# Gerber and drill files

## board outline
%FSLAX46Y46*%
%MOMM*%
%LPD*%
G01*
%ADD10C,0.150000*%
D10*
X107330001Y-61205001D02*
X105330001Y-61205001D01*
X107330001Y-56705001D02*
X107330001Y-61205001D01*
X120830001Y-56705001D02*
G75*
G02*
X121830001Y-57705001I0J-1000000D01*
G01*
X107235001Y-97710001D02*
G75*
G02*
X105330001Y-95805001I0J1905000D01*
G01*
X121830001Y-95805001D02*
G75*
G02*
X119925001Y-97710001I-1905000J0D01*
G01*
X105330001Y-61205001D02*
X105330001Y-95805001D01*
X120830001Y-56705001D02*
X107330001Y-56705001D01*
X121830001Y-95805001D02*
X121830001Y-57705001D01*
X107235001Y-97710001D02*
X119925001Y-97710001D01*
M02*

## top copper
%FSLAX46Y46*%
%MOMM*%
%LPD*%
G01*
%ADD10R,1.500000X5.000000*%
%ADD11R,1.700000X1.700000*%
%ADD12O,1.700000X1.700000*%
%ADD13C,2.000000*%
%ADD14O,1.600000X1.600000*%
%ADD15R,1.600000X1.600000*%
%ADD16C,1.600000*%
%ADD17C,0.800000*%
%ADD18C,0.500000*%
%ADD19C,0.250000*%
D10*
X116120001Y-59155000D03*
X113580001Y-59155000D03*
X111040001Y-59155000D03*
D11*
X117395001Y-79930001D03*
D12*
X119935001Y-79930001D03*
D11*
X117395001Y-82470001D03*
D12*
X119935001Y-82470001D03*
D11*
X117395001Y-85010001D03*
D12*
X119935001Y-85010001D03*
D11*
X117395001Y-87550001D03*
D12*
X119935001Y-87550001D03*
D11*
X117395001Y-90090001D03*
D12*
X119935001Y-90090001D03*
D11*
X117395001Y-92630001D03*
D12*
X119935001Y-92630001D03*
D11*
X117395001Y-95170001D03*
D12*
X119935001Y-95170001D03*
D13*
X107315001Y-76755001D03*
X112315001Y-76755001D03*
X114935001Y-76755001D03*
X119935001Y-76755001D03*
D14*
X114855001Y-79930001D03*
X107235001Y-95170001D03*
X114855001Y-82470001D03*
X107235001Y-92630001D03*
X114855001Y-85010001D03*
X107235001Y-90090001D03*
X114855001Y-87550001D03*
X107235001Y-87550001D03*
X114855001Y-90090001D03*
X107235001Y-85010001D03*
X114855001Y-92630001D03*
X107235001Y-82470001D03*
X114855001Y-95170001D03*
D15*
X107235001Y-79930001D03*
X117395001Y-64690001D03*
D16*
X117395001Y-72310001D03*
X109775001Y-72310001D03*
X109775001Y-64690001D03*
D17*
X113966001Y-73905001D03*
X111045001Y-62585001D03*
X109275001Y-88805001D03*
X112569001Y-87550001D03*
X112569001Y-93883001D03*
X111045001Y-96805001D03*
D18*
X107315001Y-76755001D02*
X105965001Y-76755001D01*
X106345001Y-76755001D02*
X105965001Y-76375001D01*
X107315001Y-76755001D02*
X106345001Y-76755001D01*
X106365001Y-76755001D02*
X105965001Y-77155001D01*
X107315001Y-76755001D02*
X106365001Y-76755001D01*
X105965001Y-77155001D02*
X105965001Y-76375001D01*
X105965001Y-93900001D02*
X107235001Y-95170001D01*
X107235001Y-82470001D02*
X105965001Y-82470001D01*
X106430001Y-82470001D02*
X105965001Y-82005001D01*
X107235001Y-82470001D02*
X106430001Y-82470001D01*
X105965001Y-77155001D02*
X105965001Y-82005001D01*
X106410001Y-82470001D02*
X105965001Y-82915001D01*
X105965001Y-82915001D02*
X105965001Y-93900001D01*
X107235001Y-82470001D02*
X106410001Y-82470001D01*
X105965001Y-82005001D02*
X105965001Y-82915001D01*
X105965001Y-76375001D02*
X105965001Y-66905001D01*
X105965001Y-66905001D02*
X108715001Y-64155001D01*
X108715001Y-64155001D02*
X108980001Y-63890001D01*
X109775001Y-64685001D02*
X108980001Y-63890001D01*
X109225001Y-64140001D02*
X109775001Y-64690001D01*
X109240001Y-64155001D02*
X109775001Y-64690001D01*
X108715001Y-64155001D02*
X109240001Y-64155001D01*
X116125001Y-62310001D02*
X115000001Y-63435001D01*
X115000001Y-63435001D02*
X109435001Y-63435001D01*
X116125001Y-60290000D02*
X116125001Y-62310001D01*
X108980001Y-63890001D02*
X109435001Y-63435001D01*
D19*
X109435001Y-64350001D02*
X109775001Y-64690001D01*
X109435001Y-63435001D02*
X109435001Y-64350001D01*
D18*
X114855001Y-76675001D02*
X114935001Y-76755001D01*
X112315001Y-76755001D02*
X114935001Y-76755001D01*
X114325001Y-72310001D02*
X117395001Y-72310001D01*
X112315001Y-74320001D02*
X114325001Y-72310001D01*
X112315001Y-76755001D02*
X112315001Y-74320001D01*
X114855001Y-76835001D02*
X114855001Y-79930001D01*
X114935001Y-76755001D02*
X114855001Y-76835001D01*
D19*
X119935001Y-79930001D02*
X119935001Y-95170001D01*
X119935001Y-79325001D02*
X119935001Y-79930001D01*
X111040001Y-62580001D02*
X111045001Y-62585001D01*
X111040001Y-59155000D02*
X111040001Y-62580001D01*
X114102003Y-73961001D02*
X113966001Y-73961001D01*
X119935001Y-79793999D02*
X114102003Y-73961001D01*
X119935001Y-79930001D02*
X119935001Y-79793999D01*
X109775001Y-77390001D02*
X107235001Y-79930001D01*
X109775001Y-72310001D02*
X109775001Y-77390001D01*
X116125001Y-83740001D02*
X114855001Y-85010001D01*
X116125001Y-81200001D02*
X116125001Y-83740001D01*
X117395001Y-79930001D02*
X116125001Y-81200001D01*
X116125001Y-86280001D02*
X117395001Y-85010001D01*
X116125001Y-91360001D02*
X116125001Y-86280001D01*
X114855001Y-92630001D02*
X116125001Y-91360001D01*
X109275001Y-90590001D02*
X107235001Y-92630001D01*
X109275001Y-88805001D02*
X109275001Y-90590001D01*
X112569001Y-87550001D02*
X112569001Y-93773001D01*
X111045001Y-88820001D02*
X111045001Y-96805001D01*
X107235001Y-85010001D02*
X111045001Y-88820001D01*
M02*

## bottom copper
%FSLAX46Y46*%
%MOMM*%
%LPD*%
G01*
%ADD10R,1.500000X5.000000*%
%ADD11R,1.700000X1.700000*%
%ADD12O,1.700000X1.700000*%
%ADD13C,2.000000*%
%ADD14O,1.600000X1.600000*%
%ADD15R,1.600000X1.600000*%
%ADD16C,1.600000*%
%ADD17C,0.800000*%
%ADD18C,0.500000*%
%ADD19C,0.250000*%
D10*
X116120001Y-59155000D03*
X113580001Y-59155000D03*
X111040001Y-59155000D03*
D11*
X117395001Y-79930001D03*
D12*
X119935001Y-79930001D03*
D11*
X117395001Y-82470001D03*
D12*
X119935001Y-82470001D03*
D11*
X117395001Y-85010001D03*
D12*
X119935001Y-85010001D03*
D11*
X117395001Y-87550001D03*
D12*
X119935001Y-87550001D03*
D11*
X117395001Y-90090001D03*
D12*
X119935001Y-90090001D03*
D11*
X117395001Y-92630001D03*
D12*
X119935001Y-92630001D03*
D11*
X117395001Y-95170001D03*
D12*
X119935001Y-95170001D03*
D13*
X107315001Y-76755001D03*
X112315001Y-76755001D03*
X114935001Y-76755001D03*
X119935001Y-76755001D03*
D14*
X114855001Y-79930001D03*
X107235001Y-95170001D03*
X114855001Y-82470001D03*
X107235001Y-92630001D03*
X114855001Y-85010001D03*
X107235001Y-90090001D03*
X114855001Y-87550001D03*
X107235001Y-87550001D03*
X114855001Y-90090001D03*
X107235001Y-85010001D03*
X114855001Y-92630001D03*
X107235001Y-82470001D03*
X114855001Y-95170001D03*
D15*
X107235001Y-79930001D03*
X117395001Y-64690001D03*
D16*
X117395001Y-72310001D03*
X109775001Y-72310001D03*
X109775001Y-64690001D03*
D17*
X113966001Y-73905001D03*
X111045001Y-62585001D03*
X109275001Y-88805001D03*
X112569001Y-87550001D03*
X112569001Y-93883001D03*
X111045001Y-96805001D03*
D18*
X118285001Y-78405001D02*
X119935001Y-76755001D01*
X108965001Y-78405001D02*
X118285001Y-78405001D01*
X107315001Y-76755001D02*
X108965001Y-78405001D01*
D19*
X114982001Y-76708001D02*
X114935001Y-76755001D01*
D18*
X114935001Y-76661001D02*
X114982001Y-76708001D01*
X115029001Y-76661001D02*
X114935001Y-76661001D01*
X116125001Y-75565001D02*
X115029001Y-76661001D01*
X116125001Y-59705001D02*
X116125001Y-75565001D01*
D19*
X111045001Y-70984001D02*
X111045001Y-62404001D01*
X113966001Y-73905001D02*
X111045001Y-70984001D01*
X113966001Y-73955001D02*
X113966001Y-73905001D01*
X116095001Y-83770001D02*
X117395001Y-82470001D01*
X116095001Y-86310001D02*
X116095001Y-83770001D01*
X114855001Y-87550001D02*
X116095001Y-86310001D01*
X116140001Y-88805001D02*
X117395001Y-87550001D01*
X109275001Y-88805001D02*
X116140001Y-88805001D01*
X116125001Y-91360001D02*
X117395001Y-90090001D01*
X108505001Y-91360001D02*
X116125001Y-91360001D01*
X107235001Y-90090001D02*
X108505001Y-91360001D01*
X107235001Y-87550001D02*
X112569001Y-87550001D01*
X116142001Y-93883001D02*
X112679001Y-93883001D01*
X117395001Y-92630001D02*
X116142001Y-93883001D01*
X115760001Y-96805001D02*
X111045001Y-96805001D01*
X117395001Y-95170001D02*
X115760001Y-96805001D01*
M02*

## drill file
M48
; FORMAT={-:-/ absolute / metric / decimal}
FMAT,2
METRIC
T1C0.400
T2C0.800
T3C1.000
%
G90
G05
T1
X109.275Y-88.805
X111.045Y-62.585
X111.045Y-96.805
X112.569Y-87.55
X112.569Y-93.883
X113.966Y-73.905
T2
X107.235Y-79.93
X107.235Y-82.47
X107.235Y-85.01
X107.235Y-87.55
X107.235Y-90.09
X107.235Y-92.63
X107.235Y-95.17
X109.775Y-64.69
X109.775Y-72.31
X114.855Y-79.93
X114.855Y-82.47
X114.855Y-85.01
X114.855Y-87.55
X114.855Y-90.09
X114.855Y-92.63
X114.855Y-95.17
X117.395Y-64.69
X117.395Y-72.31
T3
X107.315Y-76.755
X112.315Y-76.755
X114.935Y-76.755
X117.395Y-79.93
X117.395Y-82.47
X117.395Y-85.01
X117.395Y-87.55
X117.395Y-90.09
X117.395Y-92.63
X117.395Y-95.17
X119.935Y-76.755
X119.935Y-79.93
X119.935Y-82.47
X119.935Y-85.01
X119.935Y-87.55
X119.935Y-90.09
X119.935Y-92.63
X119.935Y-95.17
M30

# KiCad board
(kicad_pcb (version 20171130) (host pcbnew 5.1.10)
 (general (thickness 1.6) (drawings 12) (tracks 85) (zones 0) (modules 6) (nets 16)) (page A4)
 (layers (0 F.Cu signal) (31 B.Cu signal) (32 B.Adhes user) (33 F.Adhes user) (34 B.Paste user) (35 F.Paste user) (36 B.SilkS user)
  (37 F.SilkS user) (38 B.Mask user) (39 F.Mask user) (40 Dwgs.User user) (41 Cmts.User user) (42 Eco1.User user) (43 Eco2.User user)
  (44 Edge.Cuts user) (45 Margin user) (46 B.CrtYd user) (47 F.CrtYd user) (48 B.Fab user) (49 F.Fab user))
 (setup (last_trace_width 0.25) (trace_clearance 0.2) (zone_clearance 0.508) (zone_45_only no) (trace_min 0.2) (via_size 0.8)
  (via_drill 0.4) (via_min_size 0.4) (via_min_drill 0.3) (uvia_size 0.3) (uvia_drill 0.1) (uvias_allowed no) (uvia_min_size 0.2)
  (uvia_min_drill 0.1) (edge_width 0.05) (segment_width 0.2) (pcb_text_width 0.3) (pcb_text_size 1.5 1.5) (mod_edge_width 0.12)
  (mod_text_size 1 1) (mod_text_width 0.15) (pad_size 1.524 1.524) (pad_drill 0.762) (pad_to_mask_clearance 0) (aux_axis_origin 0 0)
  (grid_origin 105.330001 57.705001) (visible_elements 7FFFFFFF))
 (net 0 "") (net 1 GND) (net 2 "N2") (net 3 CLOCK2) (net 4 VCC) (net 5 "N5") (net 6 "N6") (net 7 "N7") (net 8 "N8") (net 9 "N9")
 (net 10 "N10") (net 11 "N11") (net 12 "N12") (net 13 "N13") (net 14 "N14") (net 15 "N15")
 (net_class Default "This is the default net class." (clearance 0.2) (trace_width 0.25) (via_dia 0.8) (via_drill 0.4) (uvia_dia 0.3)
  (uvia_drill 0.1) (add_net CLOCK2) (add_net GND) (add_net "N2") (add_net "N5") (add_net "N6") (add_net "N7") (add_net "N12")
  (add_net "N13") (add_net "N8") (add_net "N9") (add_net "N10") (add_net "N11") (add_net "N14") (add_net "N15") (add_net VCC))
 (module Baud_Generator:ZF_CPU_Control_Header (layer F.Cu) (at 113.580001 59.155 180)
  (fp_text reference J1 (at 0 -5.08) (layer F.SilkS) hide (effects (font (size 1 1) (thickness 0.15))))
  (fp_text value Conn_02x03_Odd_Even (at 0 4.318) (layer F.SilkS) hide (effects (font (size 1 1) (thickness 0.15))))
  (pad 1 connect rect (at -2.54 0) (size 1.5 5) (layers F.Cu) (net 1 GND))
  (pad 3 connect rect (at 0 0) (size 1.5 5) (layers F.Cu) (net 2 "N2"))
  (pad 5 connect rect (at 2.54 0) (size 1.5 5) (layers F.Cu) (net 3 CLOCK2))
  (pad 2 connect rect (at -2.54 0) (size 1.5 5) (layers B.Cu) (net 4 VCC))
  (pad 4 connect rect (at 0 0) (size 1.5 5) (layers B.Cu) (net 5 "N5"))
  (pad 6 connect rect (at 2.54 0) (size 1.5 5) (layers B.Cu) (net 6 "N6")))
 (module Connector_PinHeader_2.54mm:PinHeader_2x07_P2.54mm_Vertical (layer F.Cu) (at 117.395001 79.930001)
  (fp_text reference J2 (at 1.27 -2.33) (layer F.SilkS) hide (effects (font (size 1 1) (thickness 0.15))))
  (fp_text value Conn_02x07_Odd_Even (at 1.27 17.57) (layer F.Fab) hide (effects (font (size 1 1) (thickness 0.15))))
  (pad 1 thru_hole rect (at 0 0) (size 1.7 1.7) (drill 1) (layers *.Cu *.Mask) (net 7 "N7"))
  (pad 2 thru_hole oval (at 2.54 0) (size 1.7 1.7) (drill 1) (layers *.Cu *.Mask) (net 3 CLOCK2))
  (pad 3 thru_hole rect (at 0 2.54) (size 1.7 1.7) (drill 1) (layers *.Cu *.Mask) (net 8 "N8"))
  (pad 4 thru_hole oval (at 2.54 2.54) (size 1.7 1.7) (drill 1) (layers *.Cu *.Mask) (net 3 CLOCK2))
  (pad 5 thru_hole rect (at 0 5.08) (size 1.7 1.7) (drill 1) (layers *.Cu *.Mask) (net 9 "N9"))
  (pad 6 thru_hole oval (at 2.54 5.08) (size 1.7 1.7) (drill 1) (layers *.Cu *.Mask) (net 3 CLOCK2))
  (pad 7 thru_hole rect (at 0 7.62) (size 1.7 1.7) (drill 1) (layers *.Cu *.Mask) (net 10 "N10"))
  (pad 8 thru_hole oval (at 2.54 7.62) (size 1.7 1.7) (drill 1) (layers *.Cu *.Mask) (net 3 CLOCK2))
  (pad 9 thru_hole rect (at 0 10.16) (size 1.7 1.7) (drill 1) (layers *.Cu *.Mask) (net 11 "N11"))
  (pad 10 thru_hole oval (at 2.54 10.16) (size 1.7 1.7) (drill 1) (layers *.Cu *.Mask) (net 3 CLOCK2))
  (pad 11 thru_hole rect (at 0 12.7) (size 1.7 1.7) (drill 1) (layers *.Cu *.Mask) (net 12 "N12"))
  (pad 12 thru_hole oval (at 2.54 12.7) (size 1.7 1.7) (drill 1) (layers *.Cu *.Mask) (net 3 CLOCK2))
  (pad 13 thru_hole rect (at 0 15.24) (size 1.7 1.7) (drill 1) (layers *.Cu *.Mask) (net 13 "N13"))
  (pad 14 thru_hole oval (at 2.54 15.24) (size 1.7 1.7) (drill 1) (layers *.Cu *.Mask) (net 3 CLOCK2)))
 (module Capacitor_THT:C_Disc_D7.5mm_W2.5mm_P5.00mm (layer F.Cu) (at 112.315001 76.755001 180)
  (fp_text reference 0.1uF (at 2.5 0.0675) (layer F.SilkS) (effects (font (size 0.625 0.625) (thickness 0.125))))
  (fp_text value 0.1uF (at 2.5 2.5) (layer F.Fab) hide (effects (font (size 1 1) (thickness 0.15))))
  (pad 2 thru_hole circle (at 5 0 180) (size 2 2) (drill 1) (layers *.Cu *.Mask) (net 1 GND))
  (pad 1 thru_hole circle (at 0 0 180) (size 2 2) (drill 1) (layers *.Cu *.Mask) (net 4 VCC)))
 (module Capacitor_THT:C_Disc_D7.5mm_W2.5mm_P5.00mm (layer F.Cu) (at 114.935001 76.755001)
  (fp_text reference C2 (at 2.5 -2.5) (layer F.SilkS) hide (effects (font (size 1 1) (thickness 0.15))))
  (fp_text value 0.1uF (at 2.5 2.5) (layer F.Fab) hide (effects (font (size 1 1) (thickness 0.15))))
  (pad 1 thru_hole circle (at 0 0) (size 2 2) (drill 1) (layers *.Cu *.Mask) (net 4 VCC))
  (pad 2 thru_hole circle (at 5 0) (size 2 2) (drill 1) (layers *.Cu *.Mask) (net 1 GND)))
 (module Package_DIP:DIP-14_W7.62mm (layer F.Cu) (at 107.235001 79.930001)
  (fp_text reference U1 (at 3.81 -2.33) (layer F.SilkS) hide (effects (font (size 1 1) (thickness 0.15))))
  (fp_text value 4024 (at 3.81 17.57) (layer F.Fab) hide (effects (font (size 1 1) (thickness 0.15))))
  (pad 14 thru_hole oval (at 7.62 0) (size 1.6 1.6) (drill 0.8) (layers *.Cu *.Mask) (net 4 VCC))
  (pad 7 thru_hole oval (at 0 15.24) (size 1.6 1.6) (drill 0.8) (layers *.Cu *.Mask) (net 1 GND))
  (pad 13 thru_hole oval (at 7.62 2.54) (size 1.6 1.6) (drill 0.8) (layers *.Cu *.Mask))
  (pad 6 thru_hole oval (at 0 12.7) (size 1.6 1.6) (drill 0.8) (layers *.Cu *.Mask) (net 10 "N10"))
  (pad 12 thru_hole oval (at 7.62 5.08) (size 1.6 1.6) (drill 0.8) (layers *.Cu *.Mask) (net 7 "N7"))
  (pad 5 thru_hole oval (at 0 10.16) (size 1.6 1.6) (drill 0.8) (layers *.Cu *.Mask) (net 11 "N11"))
  (pad 11 thru_hole oval (at 7.62 7.62) (size 1.6 1.6) (drill 0.8) (layers *.Cu *.Mask) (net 8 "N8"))
  (pad 4 thru_hole oval (at 0 7.62) (size 1.6 1.6) (drill 0.8) (layers *.Cu *.Mask) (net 12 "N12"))
  (pad 10 thru_hole oval (at 7.62 10.16) (size 1.6 1.6) (drill 0.8) (layers *.Cu *.Mask))
  (pad 3 thru_hole oval (at 0 5.08) (size 1.6 1.6) (drill 0.8) (layers *.Cu *.Mask) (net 13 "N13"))
  (pad 9 thru_hole oval (at 7.62 12.7) (size 1.6 1.6) (drill 0.8) (layers *.Cu *.Mask) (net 9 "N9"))
  (pad 2 thru_hole oval (at 0 2.54) (size 1.6 1.6) (drill 0.8) (layers *.Cu *.Mask) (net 1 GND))
  (pad 8 thru_hole oval (at 7.62 15.24) (size 1.6 1.6) (drill 0.8) (layers *.Cu *.Mask))
  (pad 1 thru_hole rect (at 0 0) (size 1.6 1.6) (drill 0.8) (layers *.Cu *.Mask) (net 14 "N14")))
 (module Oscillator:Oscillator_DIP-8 (layer F.Cu) (at 117.395001 64.690001 180)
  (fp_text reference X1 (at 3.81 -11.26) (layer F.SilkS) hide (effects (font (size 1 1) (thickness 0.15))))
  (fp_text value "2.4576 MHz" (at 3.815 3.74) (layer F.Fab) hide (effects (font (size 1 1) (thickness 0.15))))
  (pad 1 thru_hole rect (at 0 0 180) (size 1.6 1.6) (drill 0.8) (layers *.Cu *.Mask) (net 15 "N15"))
  (pad 8 thru_hole circle (at 0 -7.62 180) (size 1.6 1.6) (drill 0.8) (layers *.Cu *.Mask) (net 4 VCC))
  (pad 5 thru_hole circle (at 7.62 -7.62 180) (size 1.6 1.6) (drill 0.8) (layers *.Cu *.Mask) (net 14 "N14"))
  (pad 4 thru_hole circle (at 7.62 0 180) (size 1.6 1.6) (drill 0.8) (layers *.Cu *.Mask) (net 1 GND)))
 (gr_line (start 107.330001 61.205001) (end 105.330001 61.205001) (layer Edge.Cuts) (width 0.15))
 (gr_line (start 107.330001 56.705001) (end 107.330001 61.205001) (layer Edge.Cuts) (width 0.15))
 (gr_arc (start 120.830001 57.705001) (end 121.830001 57.705001) (angle -90) (layer Edge.Cuts) (width 0.15))
 (gr_arc (start 107.235001 95.805001) (end 105.330001 95.805001) (angle -90) (layer Edge.Cuts) (width 0.15))
 (gr_arc (start 119.925001 95.805001) (end 119.925001 97.710001) (angle -90) (layer Edge.Cuts) (width 0.15))
 (gr_line (start 105.330001 61.205001) (end 105.330001 95.805001) (layer Edge.Cuts) (width 0.15))
 (gr_line (start 120.830001 56.705001) (end 107.330001 56.705001) (layer Edge.Cuts) (width 0.15))
 (gr_line (start 121.830001 95.805001) (end 121.830001 57.705001) (layer Edge.Cuts) (width 0.15))
 (gr_line (start 107.235001 97.710001) (end 119.925001 97.710001) (layer Edge.Cuts) (width 0.15))
 (segment (start 107.315001 76.755001) (end 105.965001 76.755001) (width 0.5) (layer F.Cu) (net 1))
 (segment (start 106.345001 76.755001) (end 105.965001 76.375001) (width 0.5) (layer F.Cu) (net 1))
 (segment (start 107.315001 76.755001) (end 106.345001 76.755001) (width 0.5) (layer F.Cu) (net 1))
 (segment (start 106.365001 76.755001) (end 105.965001 77.155001) (width 0.5) (layer F.Cu) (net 1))
 (segment (start 107.315001 76.755001) (end 106.365001 76.755001) (width 0.5) (layer F.Cu) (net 1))
 (segment (start 105.965001 77.155001) (end 105.965001 76.375001) (width 0.5) (layer F.Cu) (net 1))
 (segment (start 105.965001 93.900001) (end 107.235001 95.170001) (width 0.5) (layer F.Cu) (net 1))
 (segment (start 107.235001 82.470001) (end 105.965001 82.470001) (width 0.5) (layer F.Cu) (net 1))
 (segment (start 106.430001 82.470001) (end 105.965001 82.005001) (width 0.5) (layer F.Cu) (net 1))
 (segment (start 107.235001 82.470001) (end 106.430001 82.470001) (width 0.5) (layer F.Cu) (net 1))
 (segment (start 105.965001 77.155001) (end 105.965001 82.005001) (width 0.5) (layer F.Cu) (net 1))
 (segment (start 106.410001 82.470001) (end 105.965001 82.915001) (width 0.5) (layer F.Cu) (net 1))
 (segment (start 105.965001 82.915001) (end 105.965001 93.900001) (width 0.5) (layer F.Cu) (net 1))
 (segment (start 107.235001 82.470001) (end 106.410001 82.470001) (width 0.5) (layer F.Cu) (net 1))
 (segment (start 105.965001 82.005001) (end 105.965001 82.915001) (width 0.5) (layer F.Cu) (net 1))
 (segment (start 105.965001 76.375001) (end 105.965001 66.905001) (width 0.5) (layer F.Cu) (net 1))
 (segment (start 105.965001 66.905001) (end 108.715001 64.155001) (width 0.5) (layer F.Cu) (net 1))
 (segment (start 108.715001 64.155001) (end 108.980001 63.890001) (width 0.5) (layer F.Cu) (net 1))
 (segment (start 109.775001 64.685001) (end 108.980001 63.890001) (width 0.5) (layer F.Cu) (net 1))
 (segment (start 109.225001 64.140001) (end 109.775001 64.690001) (width 0.5) (layer F.Cu) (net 1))
 (segment (start 109.240001 64.155001) (end 109.775001 64.690001) (width 0.5) (layer F.Cu) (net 1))
 (segment (start 108.715001 64.155001) (end 109.240001 64.155001) (width 0.5) (layer F.Cu) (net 1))
 (segment (start 118.285001 78.405001) (end 119.935001 76.755001) (width 0.5) (layer B.Cu) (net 1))
 (segment (start 108.965001 78.405001) (end 118.285001 78.405001) (width 0.5) (layer B.Cu) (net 1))
 (segment (start 107.315001 76.755001) (end 108.965001 78.405001) (width 0.5) (layer B.Cu) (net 1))
 (segment (start 116.125001 62.310001) (end 115.000001 63.435001) (width 0.5) (layer F.Cu) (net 1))
 (segment (start 115.000001 63.435001) (end 109.435001 63.435001) (width 0.5) (layer F.Cu) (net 1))
 (segment (start 116.125001 60.29) (end 116.125001 62.310001) (width 0.5) (layer F.Cu) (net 1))
 (segment (start 108.980001 63.890001) (end 109.435001 63.435001) (width 0.5) (layer F.Cu) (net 1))
 (segment (start 109.435001 64.350001) (end 109.775001 64.690001) (width 0.25) (layer F.Cu) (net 1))
 (segment (start 109.435001 63.435001) (end 109.435001 64.350001) (width 0.25) (layer F.Cu) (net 1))
 (segment (start 114.855001 76.675001) (end 114.935001 76.755001) (width 0.5) (layer F.Cu) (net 4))
 (segment (start 112.315001 76.755001) (end 114.935001 76.755001) (width 0.5) (layer F.Cu) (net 4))
 (segment (start 114.982001 76.708001) (end 114.935001 76.755001) (width 0.25) (layer B.Cu) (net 4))
 (segment (start 114.325001 72.310001) (end 117.395001 72.310001) (width 0.5) (layer F.Cu) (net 4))
 (segment (start 112.315001 74.320001) (end 114.325001 72.310001) (width 0.5) (layer F.Cu) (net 4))
 (segment (start 112.315001 76.755001) (end 112.315001 74.320001) (width 0.5) (layer F.Cu) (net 4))
 (segment (start 114.935001 76.661001) (end 114.982001 76.708001) (width 0.5) (layer B.Cu) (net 4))
 (segment (start 115.029001 76.661001) (end 114.935001 76.661001) (width 0.5) (layer B.Cu) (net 4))
 (segment (start 116.125001 75.565001) (end 115.029001 76.661001) (width 0.5) (layer B.Cu) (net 4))
 (segment (start 116.125001 59.705001) (end 116.125001 75.565001) (width 0.5) (layer B.Cu) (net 4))
 (segment (start 114.855001 76.835001) (end 114.855001 79.930001) (width 0.5) (layer F.Cu) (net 4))
 (segment (start 114.935001 76.755001) (end 114.855001 76.835001) (width 0.5) (layer F.Cu) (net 4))
 (segment (start 119.935001 79.930001) (end 119.935001 95.170001) (width 0.25) (layer F.Cu) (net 3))
 (segment (start 119.935001 79.325001) (end 119.935001 79.930001) (width 0.25) (layer F.Cu) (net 3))
 (via (at 113.966001 73.905001) (size 0.8) (drill 0.4) (layers F.Cu B.Cu) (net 3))
 (via (at 111.045001 62.585001) (size 0.8) (drill 0.4) (layers F.Cu B.Cu) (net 3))
 (segment (start 111.040001 62.580001) (end 111.045001 62.585001) (width 0.25) (layer F.Cu) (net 3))
 (segment (start 111.040001 59.155) (end 111.040001 62.580001) (width 0.25) (layer F.Cu) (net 3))
 (segment (start 114.102003 73.961001) (end 113.966001 73.961001) (width 0.25) (layer F.Cu) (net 3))
 (segment (start 119.935001 79.793999) (end 114.102003 73.961001) (width 0.25) (layer F.Cu) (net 3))
 (segment (start 119.935001 79.930001) (end 119.935001 79.793999) (width 0.25) (layer F.Cu) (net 3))
 (segment (start 111.045001 70.984001) (end 111.045001 62.404001) (width 0.25) (layer B.Cu) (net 3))
 (segment (start 113.966001 73.905001) (end 111.045001 70.984001) (width 0.25) (layer B.Cu) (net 3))
 (segment (start 113.966001 73.955001) (end 113.966001 73.905001) (width 0.25) (layer B.Cu) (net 3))
 (segment (start 109.775001 77.390001) (end 107.235001 79.930001) (width 0.25) (layer F.Cu) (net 14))
 (segment (start 109.775001 72.310001) (end 109.775001 77.390001) (width 0.25) (layer F.Cu) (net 14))
 (segment (start 116.125001 83.740001) (end 114.855001 85.010001) (width 0.25) (layer F.Cu) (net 7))
 (segment (start 116.125001 81.200001) (end 116.125001 83.740001) (width 0.25) (layer F.Cu) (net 7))
 (segment (start 117.395001 79.930001) (end 116.125001 81.200001) (width 0.25) (layer F.Cu) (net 7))
 (segment (start 116.095001 83.770001) (end 117.395001 82.470001) (width 0.25) (layer B.Cu) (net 8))
 (segment (start 116.095001 86.310001) (end 116.095001 83.770001) (width 0.25) (layer B.Cu) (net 8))
 (segment (start 114.855001 87.550001) (end 116.095001 86.310001) (width 0.25) (layer B.Cu) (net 8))
 (segment (start 116.125001 86.280001) (end 117.395001 85.010001) (width 0.25) (layer F.Cu) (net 9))
 (segment (start 116.125001 91.360001) (end 116.125001 86.280001) (width 0.25) (layer F.Cu) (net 9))
 (segment (start 114.855001 92.630001) (end 116.125001 91.360001) (width 0.25) (layer F.Cu) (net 9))
 (via (at 109.275001 88.805001) (size 0.8) (drill 0.4) (layers F.Cu B.Cu) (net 10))
 (segment (start 116.140001 88.805001) (end 117.395001 87.550001) (width 0.25) (layer B.Cu) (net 10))
 (segment (start 109.275001 88.805001) (end 116.140001 88.805001) (width 0.25) (layer B.Cu) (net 10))
 (segment (start 109.275001 90.590001) (end 107.235001 92.630001) (width 0.25) (layer F.Cu) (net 10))
 (segment (start 109.275001 88.805001) (end 109.275001 90.590001) (width 0.25) (layer F.Cu) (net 10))
 (segment (start 116.125001 91.360001) (end 117.395001 90.090001) (width 0.25) (layer B.Cu) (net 11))
 (segment (start 108.505001 91.360001) (end 116.125001 91.360001) (width 0.25) (layer B.Cu) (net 11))
 (segment (start 107.235001 90.090001) (end 108.505001 91.360001) (width 0.25) (layer B.Cu) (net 11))
 (via (at 112.569001 87.550001) (size 0.8) (drill 0.4) (layers F.Cu B.Cu) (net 12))
 (via (at 112.569001 93.883001) (size 0.8) (drill 0.4) (layers F.Cu B.Cu) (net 12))
 (segment (start 112.569001 87.550001) (end 112.569001 93.773001) (width 0.25) (layer F.Cu) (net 12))
 (segment (start 107.235001 87.550001) (end 112.569001 87.550001) (width 0.25) (layer B.Cu) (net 12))
 (segment (start 116.142001 93.883001) (end 112.679001 93.883001) (width 0.25) (layer B.Cu) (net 12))
 (segment (start 117.395001 92.630001) (end 116.142001 93.883001) (width 0.25) (layer B.Cu) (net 12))
 (via (at 111.045001 96.805001) (size 0.8) (drill 0.4) (layers F.Cu B.Cu) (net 13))
 (segment (start 111.045001 88.820001) (end 111.045001 96.805001) (width 0.25) (layer F.Cu) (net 13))
 (segment (start 107.235001 85.010001) (end 111.045001 88.820001) (width 0.25) (layer F.Cu) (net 13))
 (segment (start 115.760001 96.805001) (end 111.045001 96.805001) (width 0.25) (layer B.Cu) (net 13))
 (segment (start 117.395001 95.170001) (end 115.760001 96.805001) (width 0.25) (layer B.Cu) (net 13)))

